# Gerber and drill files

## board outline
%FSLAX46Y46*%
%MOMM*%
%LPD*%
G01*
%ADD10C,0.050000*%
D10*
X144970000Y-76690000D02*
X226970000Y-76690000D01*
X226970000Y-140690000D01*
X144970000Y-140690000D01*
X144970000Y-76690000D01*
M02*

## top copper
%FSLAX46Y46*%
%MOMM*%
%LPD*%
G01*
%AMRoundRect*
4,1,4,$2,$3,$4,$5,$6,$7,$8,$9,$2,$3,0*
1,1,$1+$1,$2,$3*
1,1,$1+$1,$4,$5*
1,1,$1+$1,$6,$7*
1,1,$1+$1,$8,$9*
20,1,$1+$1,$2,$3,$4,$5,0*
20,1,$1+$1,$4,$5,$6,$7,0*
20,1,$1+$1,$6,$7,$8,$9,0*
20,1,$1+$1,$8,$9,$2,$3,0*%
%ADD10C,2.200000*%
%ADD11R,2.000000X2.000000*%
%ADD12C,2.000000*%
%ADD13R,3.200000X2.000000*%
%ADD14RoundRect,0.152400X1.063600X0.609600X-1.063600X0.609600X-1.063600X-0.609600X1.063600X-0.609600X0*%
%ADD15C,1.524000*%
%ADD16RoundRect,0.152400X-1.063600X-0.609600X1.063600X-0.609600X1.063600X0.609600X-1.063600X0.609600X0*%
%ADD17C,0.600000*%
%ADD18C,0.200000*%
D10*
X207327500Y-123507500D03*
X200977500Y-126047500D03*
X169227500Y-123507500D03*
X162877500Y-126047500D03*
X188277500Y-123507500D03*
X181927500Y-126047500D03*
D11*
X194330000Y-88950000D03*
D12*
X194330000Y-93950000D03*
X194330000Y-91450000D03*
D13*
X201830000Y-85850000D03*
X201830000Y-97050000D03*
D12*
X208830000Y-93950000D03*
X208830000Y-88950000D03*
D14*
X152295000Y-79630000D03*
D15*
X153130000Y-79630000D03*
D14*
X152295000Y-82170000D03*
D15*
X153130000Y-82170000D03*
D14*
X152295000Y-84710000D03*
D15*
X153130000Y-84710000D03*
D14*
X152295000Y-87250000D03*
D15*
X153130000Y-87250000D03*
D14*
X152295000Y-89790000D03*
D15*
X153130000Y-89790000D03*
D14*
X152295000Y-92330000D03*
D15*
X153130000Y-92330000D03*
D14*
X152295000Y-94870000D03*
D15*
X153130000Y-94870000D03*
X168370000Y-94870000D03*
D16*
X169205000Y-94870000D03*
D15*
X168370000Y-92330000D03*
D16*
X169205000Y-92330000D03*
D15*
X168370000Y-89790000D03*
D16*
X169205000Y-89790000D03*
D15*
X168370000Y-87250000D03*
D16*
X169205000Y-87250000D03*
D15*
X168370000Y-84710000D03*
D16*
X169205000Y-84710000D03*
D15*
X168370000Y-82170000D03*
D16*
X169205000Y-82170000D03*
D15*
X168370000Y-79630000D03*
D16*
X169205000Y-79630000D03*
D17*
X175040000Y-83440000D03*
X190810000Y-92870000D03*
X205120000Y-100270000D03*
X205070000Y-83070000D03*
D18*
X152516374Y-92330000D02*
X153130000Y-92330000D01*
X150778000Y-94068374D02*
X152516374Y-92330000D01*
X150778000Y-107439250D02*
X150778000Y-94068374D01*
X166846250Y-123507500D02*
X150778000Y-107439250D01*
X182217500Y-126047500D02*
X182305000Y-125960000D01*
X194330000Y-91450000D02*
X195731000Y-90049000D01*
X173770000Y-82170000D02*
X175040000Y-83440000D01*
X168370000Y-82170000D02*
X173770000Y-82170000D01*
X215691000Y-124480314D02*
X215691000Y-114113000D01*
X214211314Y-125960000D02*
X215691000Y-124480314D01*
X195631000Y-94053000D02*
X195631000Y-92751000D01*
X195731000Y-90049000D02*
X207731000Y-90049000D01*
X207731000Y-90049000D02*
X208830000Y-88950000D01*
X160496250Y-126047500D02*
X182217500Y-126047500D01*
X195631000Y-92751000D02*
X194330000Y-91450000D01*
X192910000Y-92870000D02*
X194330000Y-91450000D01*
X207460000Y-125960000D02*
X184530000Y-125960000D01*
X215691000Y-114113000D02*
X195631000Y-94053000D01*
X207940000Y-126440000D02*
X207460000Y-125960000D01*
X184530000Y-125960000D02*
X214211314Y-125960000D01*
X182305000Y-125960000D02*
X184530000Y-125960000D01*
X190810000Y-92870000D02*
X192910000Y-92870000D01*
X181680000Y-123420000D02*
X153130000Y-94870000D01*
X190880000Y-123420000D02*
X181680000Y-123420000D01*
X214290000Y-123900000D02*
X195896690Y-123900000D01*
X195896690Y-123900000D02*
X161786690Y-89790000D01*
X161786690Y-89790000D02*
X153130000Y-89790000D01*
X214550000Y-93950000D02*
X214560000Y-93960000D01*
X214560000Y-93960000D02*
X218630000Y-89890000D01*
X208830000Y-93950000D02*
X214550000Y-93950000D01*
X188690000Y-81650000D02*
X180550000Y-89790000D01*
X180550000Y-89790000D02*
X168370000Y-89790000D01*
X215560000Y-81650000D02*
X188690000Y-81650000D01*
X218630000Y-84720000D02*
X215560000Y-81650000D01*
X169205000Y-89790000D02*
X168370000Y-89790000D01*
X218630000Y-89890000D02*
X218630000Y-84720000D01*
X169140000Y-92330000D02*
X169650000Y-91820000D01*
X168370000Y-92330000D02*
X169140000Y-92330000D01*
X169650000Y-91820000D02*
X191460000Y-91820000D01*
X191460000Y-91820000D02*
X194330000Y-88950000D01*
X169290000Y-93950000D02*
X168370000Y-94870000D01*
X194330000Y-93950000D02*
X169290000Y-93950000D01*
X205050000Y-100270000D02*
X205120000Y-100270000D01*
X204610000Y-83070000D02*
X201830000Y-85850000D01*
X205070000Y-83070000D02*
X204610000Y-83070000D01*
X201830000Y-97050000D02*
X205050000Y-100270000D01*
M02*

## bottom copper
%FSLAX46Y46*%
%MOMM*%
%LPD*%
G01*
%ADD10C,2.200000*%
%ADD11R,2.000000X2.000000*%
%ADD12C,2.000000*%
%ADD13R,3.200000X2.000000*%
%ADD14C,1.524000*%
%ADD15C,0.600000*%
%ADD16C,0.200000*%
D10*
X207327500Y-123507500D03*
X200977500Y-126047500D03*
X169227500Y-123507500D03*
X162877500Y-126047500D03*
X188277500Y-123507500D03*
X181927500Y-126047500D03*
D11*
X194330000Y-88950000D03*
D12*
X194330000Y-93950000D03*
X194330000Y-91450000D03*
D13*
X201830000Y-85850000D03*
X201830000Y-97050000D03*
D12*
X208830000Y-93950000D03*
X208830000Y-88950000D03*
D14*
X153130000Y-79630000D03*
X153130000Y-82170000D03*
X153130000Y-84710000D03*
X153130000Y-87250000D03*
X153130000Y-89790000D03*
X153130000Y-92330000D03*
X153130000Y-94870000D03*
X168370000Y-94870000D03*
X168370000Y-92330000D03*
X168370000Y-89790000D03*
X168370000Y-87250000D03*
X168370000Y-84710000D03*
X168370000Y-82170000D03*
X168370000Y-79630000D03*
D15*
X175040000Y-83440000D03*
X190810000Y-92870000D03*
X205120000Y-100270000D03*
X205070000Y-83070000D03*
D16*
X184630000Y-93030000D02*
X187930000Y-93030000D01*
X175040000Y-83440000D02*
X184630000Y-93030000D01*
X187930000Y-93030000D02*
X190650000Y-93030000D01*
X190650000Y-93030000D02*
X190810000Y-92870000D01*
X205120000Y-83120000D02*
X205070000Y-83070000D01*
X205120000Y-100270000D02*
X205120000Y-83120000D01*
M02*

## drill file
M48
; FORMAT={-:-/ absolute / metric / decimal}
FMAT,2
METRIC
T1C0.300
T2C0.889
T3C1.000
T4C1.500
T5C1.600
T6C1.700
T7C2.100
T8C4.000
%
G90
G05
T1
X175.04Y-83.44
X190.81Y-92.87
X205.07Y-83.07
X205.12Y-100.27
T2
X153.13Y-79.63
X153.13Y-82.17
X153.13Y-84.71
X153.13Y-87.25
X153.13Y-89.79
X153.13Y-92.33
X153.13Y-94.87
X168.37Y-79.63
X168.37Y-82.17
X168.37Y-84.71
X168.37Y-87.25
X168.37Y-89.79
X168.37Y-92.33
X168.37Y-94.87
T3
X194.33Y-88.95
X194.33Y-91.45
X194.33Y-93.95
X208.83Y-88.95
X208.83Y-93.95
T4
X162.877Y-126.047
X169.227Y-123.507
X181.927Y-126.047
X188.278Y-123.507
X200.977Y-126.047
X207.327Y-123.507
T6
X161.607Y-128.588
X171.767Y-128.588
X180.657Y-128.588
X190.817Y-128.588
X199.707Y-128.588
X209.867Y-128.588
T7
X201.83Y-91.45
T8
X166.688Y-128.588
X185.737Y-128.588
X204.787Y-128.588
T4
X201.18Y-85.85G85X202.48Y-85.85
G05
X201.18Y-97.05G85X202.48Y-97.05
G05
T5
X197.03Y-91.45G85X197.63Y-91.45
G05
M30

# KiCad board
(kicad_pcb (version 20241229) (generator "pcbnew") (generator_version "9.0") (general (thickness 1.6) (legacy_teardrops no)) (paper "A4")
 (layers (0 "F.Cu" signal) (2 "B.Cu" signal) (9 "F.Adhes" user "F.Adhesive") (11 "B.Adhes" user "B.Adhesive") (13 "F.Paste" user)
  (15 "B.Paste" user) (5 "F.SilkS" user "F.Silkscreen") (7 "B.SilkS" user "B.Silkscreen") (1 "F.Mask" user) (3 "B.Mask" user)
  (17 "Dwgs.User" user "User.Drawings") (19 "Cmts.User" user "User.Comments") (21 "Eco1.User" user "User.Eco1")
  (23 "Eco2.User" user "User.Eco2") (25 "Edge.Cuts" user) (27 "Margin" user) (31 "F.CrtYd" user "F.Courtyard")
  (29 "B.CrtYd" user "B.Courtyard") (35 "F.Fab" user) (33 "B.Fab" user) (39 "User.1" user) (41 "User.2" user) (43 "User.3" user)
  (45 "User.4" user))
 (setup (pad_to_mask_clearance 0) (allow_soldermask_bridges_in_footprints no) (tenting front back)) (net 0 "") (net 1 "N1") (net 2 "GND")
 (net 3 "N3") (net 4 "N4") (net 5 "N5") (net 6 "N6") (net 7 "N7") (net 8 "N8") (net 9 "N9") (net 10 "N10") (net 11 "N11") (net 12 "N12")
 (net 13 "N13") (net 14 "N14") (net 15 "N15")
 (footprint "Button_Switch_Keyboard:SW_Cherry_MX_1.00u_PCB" (layer "F.Cu") (at 207.3275 123.5075)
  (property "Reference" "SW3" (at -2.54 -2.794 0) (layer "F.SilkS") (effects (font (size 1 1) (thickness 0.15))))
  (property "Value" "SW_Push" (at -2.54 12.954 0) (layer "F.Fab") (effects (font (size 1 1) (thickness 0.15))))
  (pad "" np_thru_hole circle (at -7.62 5.08) (size 1.7 1.7) (drill 1.7) (layers "*.Cu" "*.Mask"))
  (pad "" np_thru_hole circle (at -2.54 5.08) (size 4 4) (drill 4) (layers "*.Cu" "*.Mask"))
  (pad "" np_thru_hole circle (at 2.54 5.08) (size 1.7 1.7) (drill 1.7) (layers "*.Cu" "*.Mask"))
  (pad "1" thru_hole circle (at 0 0) (size 2.2 2.2) (drill 1.5) (layers "*.Cu" "*.Mask") (remove_unused_layers no) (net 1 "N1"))
  (pad "2" thru_hole circle (at -6.35 2.54) (size 2.2 2.2) (drill 1.5) (layers "*.Cu" "*.Mask") (remove_unused_layers no) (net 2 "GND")))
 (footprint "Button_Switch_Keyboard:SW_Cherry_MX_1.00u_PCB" (layer "F.Cu") (at 169.2275 123.5075)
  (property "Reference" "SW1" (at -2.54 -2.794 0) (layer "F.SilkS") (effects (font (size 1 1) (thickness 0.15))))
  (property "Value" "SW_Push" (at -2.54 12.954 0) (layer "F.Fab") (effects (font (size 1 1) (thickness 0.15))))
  (pad "" np_thru_hole circle (at -7.62 5.08) (size 1.7 1.7) (drill 1.7) (layers "*.Cu" "*.Mask"))
  (pad "" np_thru_hole circle (at -2.54 5.08) (size 4 4) (drill 4) (layers "*.Cu" "*.Mask"))
  (pad "" np_thru_hole circle (at 2.54 5.08) (size 1.7 1.7) (drill 1.7) (layers "*.Cu" "*.Mask"))
  (pad "1" thru_hole circle (at 0 0) (size 2.2 2.2) (drill 1.5) (layers "*.Cu" "*.Mask") (remove_unused_layers no) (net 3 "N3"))
  (pad "2" thru_hole circle (at -6.35 2.54) (size 2.2 2.2) (drill 1.5) (layers "*.Cu" "*.Mask") (remove_unused_layers no) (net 2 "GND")))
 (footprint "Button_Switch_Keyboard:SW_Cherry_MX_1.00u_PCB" (layer "F.Cu") (at 188.2775 123.5075)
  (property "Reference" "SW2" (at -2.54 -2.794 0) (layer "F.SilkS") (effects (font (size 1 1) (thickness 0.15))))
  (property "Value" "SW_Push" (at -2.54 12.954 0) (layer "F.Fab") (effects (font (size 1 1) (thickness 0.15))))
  (pad "" np_thru_hole circle (at -7.62 5.08) (size 1.7 1.7) (drill 1.7) (layers "*.Cu" "*.Mask"))
  (pad "" np_thru_hole circle (at -2.54 5.08) (size 4 4) (drill 4) (layers "*.Cu" "*.Mask"))
  (pad "" np_thru_hole circle (at 2.54 5.08) (size 1.7 1.7) (drill 1.7) (layers "*.Cu" "*.Mask"))
  (pad "1" thru_hole circle (at 0 0) (size 2.2 2.2) (drill 1.5) (layers "*.Cu" "*.Mask") (remove_unused_layers no) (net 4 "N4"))
  (pad "2" thru_hole circle (at -6.35 2.54) (size 2.2 2.2) (drill 1.5) (layers "*.Cu" "*.Mask") (remove_unused_layers no) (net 2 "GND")))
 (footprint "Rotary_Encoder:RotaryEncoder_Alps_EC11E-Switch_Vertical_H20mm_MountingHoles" (layer "F.Cu") (at 194.33 88.95)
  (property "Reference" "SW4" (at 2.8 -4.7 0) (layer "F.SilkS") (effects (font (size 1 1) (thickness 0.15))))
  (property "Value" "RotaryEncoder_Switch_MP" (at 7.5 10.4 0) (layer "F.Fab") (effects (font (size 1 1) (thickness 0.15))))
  (pad "" np_thru_hole oval (at 3 2.5) (size 2.2 1.6) (drill oval 2.2 1.6) (layers "*.Mask"))
  (pad "" np_thru_hole circle (at 7.5 2.5) (size 2.1 2.1) (drill 2.1) (layers "*.Mask"))
  (pad "A" thru_hole rect (at 0 0) (size 2 2) (drill 1) (layers "*.Cu" "*.Mask") (remove_unused_layers no) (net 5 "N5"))
  (pad "B" thru_hole circle (at 0 5) (size 2 2) (drill 1) (layers "*.Cu" "*.Mask") (remove_unused_layers no) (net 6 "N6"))
  (pad "C" thru_hole circle (at 0 2.5) (size 2 2) (drill 1) (layers "*.Cu" "*.Mask") (remove_unused_layers no) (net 2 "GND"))
  (pad "MP" thru_hole rect (at 7.5 -3.1) (size 3.2 2) (drill oval 2.8 1.5) (layers "*.Cu" "*.Mask") (remove_unused_layers no) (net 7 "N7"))
  (pad "MP" thru_hole rect (at 7.5 8.1) (size 3.2 2) (drill oval 2.8 1.5) (layers "*.Cu" "*.Mask") (remove_unused_layers no) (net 7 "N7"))
  (pad "S1" thru_hole circle (at 14.5 5) (size 2 2) (drill 1) (layers "*.Cu" "*.Mask") (remove_unused_layers no) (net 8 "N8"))
  (pad "S2" thru_hole circle (at 14.5 0) (size 2 2) (drill 1) (layers "*.Cu" "*.Mask") (remove_unused_layers no) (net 2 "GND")))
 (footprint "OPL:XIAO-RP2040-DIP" (layer "F.Cu") (at 160.75 87.25)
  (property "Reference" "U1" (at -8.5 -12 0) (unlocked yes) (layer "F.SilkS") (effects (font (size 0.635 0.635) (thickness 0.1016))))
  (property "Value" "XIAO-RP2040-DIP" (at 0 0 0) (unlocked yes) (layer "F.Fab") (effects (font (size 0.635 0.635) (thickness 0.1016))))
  (pad "1" smd roundrect (at -8.455 -7.62 180) (size 2.432 1.524) (layers "F.Cu" "F.Mask") (roundrect_rratio 0.1) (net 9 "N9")
   (thermal_bridge_angle 45))
  (pad "1" thru_hole circle (at -7.62 -7.62 180) (size 1.524 1.524) (drill 0.889) (layers "*.Cu" "*.Mask") (remove_unused_layers no)
   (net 9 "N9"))
  (pad "2" smd roundrect (at -8.455 -5.08 180) (size 2.432 1.524) (layers "F.Cu" "F.Mask") (roundrect_rratio 0.1) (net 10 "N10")
   (thermal_bridge_angle 45))
  (pad "2" thru_hole circle (at -7.62 -5.08 180) (size 1.524 1.524) (drill 0.889) (layers "*.Cu" "*.Mask") (remove_unused_layers no)
   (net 10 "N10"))
  (pad "3" smd roundrect (at -8.455 -2.54 180) (size 2.432 1.524) (layers "F.Cu" "F.Mask") (roundrect_rratio 0.1) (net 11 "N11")
   (thermal_bridge_angle 45))
  (pad "3" thru_hole circle (at -7.62 -2.54 180) (size 1.524 1.524) (drill 0.889) (layers "*.Cu" "*.Mask") (remove_unused_layers no)
   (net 11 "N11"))
  (pad "4" smd roundrect (at -8.455 0 180) (size 2.432 1.524) (layers "F.Cu" "F.Mask") (roundrect_rratio 0.1) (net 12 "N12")
   (thermal_bridge_angle 45))
  (pad "4" thru_hole circle (at -7.62 0 180) (size 1.524 1.524) (drill 0.889) (layers "*.Cu" "*.Mask") (remove_unused_layers no)
   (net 12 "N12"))
  (pad "5" smd roundrect (at -8.455 2.54 180) (size 2.432 1.524) (layers "F.Cu" "F.Mask") (roundrect_rratio 0.1) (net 1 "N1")
   (thermal_bridge_angle 45))
  (pad "5" thru_hole circle (at -7.62 2.54 180) (size 1.524 1.524) (drill 0.889) (layers "*.Cu" "*.Mask") (remove_unused_layers no)
   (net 1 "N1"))
  (pad "6" smd roundrect (at -8.455 5.08 180) (size 2.432 1.524) (layers "F.Cu" "F.Mask") (roundrect_rratio 0.1) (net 3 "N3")
   (thermal_bridge_angle 45))
  (pad "6" thru_hole circle (at -7.62 5.08 180) (size 1.524 1.524) (drill 0.889) (layers "*.Cu" "*.Mask") (remove_unused_layers no)
   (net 3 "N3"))
  (pad "7" smd roundrect (at -8.455 7.62 180) (size 2.432 1.524) (layers "F.Cu" "F.Mask") (roundrect_rratio 0.1) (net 4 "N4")
   (thermal_bridge_angle 45))
  (pad "7" thru_hole circle (at -7.62 7.62 180) (size 1.524 1.524) (drill 0.889) (layers "*.Cu" "*.Mask") (remove_unused_layers no)
   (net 4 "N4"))
  (pad "8" thru_hole circle (at 7.62 7.62) (size 1.524 1.524) (drill 0.889) (layers "*.Cu" "*.Mask") (remove_unused_layers no) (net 6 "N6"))
  (pad "8" smd roundrect (at 8.455 7.62) (size 2.432 1.524) (layers "F.Cu" "F.Mask") (roundrect_rratio 0.1) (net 6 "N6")
   (thermal_bridge_angle 45))
  (pad "9" thru_hole circle (at 7.62 5.08) (size 1.524 1.524) (drill 0.889) (layers "*.Cu" "*.Mask") (remove_unused_layers no) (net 5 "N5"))
  (pad "9" smd roundrect (at 8.455 5.08) (size 2.432 1.524) (layers "F.Cu" "F.Mask") (roundrect_rratio 0.1) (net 5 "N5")
   (thermal_bridge_angle 45))
  (pad "10" thru_hole circle (at 7.62 2.54) (size 1.524 1.524) (drill 0.889) (layers "*.Cu" "*.Mask") (remove_unused_layers no) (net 8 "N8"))
  (pad "10" smd roundrect (at 8.455 2.54) (size 2.432 1.524) (layers "F.Cu" "F.Mask") (roundrect_rratio 0.1) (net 8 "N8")
   (thermal_bridge_angle 45))
  (pad "11" thru_hole circle (at 7.62 0) (size 1.524 1.524) (drill 0.889) (layers "*.Cu" "*.Mask") (remove_unused_layers no) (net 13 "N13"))
  (pad "11" smd roundrect (at 8.455 0) (size 2.432 1.524) (layers "F.Cu" "F.Mask") (roundrect_rratio 0.1) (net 13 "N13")
   (thermal_bridge_angle 45))
  (pad "12" thru_hole circle (at 7.62 -2.54) (size 1.524 1.524) (drill 0.889) (layers "*.Cu" "*.Mask") (remove_unused_layers no)
   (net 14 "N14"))
  (pad "12" smd roundrect (at 8.455 -2.54) (size 2.432 1.524) (layers "F.Cu" "F.Mask") (roundrect_rratio 0.1) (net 14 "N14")
   (thermal_bridge_angle 45))
  (pad "13" thru_hole circle (at 7.62 -5.08) (size 1.524 1.524) (drill 0.889) (layers "*.Cu" "*.Mask") (remove_unused_layers no)
   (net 2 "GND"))
  (pad "13" smd roundrect (at 8.455 -5.08) (size 2.432 1.524) (layers "F.Cu" "F.Mask") (roundrect_rratio 0.1) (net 2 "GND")
   (thermal_bridge_angle 45))
  (pad "14" thru_hole circle (at 7.62 -7.62) (size 1.524 1.524) (drill 0.889) (layers "*.Cu" "*.Mask") (remove_unused_layers no)
   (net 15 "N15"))
  (pad "14" smd roundrect (at 8.455 -7.62) (size 2.432 1.524) (layers "F.Cu" "F.Mask") (roundrect_rratio 0.1) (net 15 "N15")
   (thermal_bridge_angle 45)))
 (gr_rect (start 144.97 76.69) (end 226.97 140.69) (stroke (width 0.05) (type default)) (fill no) (layer "Edge.Cuts"))
 (segment (start 152.516374 92.33) (end 153.13 92.33) (width 0.2) (layer "F.Cu") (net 3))
 (segment (start 150.778 94.068374) (end 152.516374 92.33) (width 0.2) (layer "F.Cu") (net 3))
 (segment (start 150.778 107.43925) (end 150.778 94.068374) (width 0.2) (layer "F.Cu") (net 3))
 (segment (start 166.84625 123.5075) (end 150.778 107.43925) (width 0.2) (layer "F.Cu") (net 3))
 (segment (start 182.2175 126.0475) (end 182.305 125.96) (width 0.2) (layer "F.Cu") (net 2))
 (segment (start 194.33 91.45) (end 195.731 90.049) (width 0.2) (layer "F.Cu") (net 2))
 (segment (start 173.77 82.17) (end 175.04 83.44) (width 0.2) (layer "F.Cu") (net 2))
 (segment (start 168.37 82.17) (end 173.77 82.17) (width 0.2) (layer "F.Cu") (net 2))
 (segment (start 215.691 124.480314) (end 215.691 114.113) (width 0.2) (layer "F.Cu") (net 2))
 (segment (start 214.211314 125.96) (end 215.691 124.480314) (width 0.2) (layer "F.Cu") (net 2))
 (segment (start 195.631 94.053) (end 195.631 92.751) (width 0.2) (layer "F.Cu") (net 2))
 (segment (start 195.731 90.049) (end 207.731 90.049) (width 0.2) (layer "F.Cu") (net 2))
 (segment (start 207.731 90.049) (end 208.83 88.95) (width 0.2) (layer "F.Cu") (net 2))
 (segment (start 160.49625 126.0475) (end 182.2175 126.0475) (width 0.2) (layer "F.Cu") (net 2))
 (segment (start 195.631 92.751) (end 194.33 91.45) (width 0.2) (layer "F.Cu") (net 2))
 (segment (start 192.91 92.87) (end 194.33 91.45) (width 0.2) (layer "F.Cu") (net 2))
 (segment (start 207.46 125.96) (end 184.53 125.96) (width 0.2) (layer "F.Cu") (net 2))
 (segment (start 215.691 114.113) (end 195.631 94.053) (width 0.2) (layer "F.Cu") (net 2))
 (segment (start 207.94 126.44) (end 207.46 125.96) (width 0.2) (layer "F.Cu") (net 2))
 (segment (start 184.53 125.96) (end 214.211314 125.96) (width 0.2) (layer "F.Cu") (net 2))
 (segment (start 182.305 125.96) (end 184.53 125.96) (width 0.2) (layer "F.Cu") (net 2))
 (segment (start 190.81 92.87) (end 192.91 92.87) (width 0.2) (layer "F.Cu") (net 2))
 (via (at 175.04 83.44) (size 0.6) (drill 0.3) (layers "F.Cu" "B.Cu") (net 2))
 (via (at 190.81 92.87) (size 0.6) (drill 0.3) (layers "F.Cu" "B.Cu") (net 2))
 (segment (start 184.63 93.03) (end 187.93 93.03) (width 0.2) (layer "B.Cu") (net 2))
 (segment (start 175.04 83.44) (end 184.63 93.03) (width 0.2) (layer "B.Cu") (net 2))
 (segment (start 187.93 93.03) (end 190.65 93.03) (width 0.2) (layer "B.Cu") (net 2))
 (segment (start 190.65 93.03) (end 190.81 92.87) (width 0.2) (layer "B.Cu") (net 2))
 (segment (start 181.68 123.42) (end 153.13 94.87) (width 0.2) (layer "F.Cu") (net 4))
 (segment (start 190.88 123.42) (end 181.68 123.42) (width 0.2) (layer "F.Cu") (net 4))
 (segment (start 214.29 123.9) (end 195.89669 123.9) (width 0.2) (layer "F.Cu") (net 1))
 (segment (start 195.89669 123.9) (end 161.78669 89.79) (width 0.2) (layer "F.Cu") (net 1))
 (segment (start 161.78669 89.79) (end 153.13 89.79) (width 0.2) (layer "F.Cu") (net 1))
 (segment (start 214.55 93.95) (end 214.56 93.96) (width 0.2) (layer "F.Cu") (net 8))
 (segment (start 214.56 93.96) (end 218.63 89.89) (width 0.2) (layer "F.Cu") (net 8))
 (segment (start 208.83 93.95) (end 214.55 93.95) (width 0.2) (layer "F.Cu") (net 8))
 (segment (start 188.69 81.65) (end 180.55 89.79) (width 0.2) (layer "F.Cu") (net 8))
 (segment (start 180.55 89.79) (end 168.37 89.79) (width 0.2) (layer "F.Cu") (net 8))
 (segment (start 215.56 81.65) (end 188.69 81.65) (width 0.2) (layer "F.Cu") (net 8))
 (segment (start 218.63 84.72) (end 215.56 81.65) (width 0.2) (layer "F.Cu") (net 8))
 (segment (start 169.205 89.79) (end 168.37 89.79) (width 0.2) (layer "F.Cu") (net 8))
 (segment (start 218.63 89.89) (end 218.63 84.72) (width 0.2) (layer "F.Cu") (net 8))
 (segment (start 169.14 92.33) (end 169.65 91.82) (width 0.2) (layer "F.Cu") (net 5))
 (segment (start 168.37 92.33) (end 169.14 92.33) (width 0.2) (layer "F.Cu") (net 5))
 (segment (start 169.65 91.82) (end 191.46 91.82) (width 0.2) (layer "F.Cu") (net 5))
 (segment (start 191.46 91.82) (end 194.33 88.95) (width 0.2) (layer "F.Cu") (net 5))
 (segment (start 169.29 93.95) (end 168.37 94.87) (width 0.2) (layer "F.Cu") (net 6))
 (segment (start 194.33 93.95) (end 169.29 93.95) (width 0.2) (layer "F.Cu") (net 6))
 (segment (start 205.05 100.27) (end 205.12 100.27) (width 0.2) (layer "F.Cu") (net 7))
 (segment (start 204.61 83.07) (end 201.83 85.85) (width 0.2) (layer "F.Cu") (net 7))
 (segment (start 205.07 83.07) (end 204.61 83.07) (width 0.2) (layer "F.Cu") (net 7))
 (segment (start 201.83 97.05) (end 205.05 100.27) (width 0.2) (layer "F.Cu") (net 7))
 (via (at 205.12 100.27) (size 0.6) (drill 0.3) (layers "F.Cu" "B.Cu") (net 7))
 (via (at 205.07 83.07) (size 0.6) (drill 0.3) (layers "F.Cu" "B.Cu") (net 7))
 (segment (start 205.12 83.12) (end 205.07 83.07) (width 0.2) (layer "B.Cu") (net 7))
 (segment (start 205.12 100.27) (end 205.12 83.12) (width 0.2) (layer "B.Cu") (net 7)))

